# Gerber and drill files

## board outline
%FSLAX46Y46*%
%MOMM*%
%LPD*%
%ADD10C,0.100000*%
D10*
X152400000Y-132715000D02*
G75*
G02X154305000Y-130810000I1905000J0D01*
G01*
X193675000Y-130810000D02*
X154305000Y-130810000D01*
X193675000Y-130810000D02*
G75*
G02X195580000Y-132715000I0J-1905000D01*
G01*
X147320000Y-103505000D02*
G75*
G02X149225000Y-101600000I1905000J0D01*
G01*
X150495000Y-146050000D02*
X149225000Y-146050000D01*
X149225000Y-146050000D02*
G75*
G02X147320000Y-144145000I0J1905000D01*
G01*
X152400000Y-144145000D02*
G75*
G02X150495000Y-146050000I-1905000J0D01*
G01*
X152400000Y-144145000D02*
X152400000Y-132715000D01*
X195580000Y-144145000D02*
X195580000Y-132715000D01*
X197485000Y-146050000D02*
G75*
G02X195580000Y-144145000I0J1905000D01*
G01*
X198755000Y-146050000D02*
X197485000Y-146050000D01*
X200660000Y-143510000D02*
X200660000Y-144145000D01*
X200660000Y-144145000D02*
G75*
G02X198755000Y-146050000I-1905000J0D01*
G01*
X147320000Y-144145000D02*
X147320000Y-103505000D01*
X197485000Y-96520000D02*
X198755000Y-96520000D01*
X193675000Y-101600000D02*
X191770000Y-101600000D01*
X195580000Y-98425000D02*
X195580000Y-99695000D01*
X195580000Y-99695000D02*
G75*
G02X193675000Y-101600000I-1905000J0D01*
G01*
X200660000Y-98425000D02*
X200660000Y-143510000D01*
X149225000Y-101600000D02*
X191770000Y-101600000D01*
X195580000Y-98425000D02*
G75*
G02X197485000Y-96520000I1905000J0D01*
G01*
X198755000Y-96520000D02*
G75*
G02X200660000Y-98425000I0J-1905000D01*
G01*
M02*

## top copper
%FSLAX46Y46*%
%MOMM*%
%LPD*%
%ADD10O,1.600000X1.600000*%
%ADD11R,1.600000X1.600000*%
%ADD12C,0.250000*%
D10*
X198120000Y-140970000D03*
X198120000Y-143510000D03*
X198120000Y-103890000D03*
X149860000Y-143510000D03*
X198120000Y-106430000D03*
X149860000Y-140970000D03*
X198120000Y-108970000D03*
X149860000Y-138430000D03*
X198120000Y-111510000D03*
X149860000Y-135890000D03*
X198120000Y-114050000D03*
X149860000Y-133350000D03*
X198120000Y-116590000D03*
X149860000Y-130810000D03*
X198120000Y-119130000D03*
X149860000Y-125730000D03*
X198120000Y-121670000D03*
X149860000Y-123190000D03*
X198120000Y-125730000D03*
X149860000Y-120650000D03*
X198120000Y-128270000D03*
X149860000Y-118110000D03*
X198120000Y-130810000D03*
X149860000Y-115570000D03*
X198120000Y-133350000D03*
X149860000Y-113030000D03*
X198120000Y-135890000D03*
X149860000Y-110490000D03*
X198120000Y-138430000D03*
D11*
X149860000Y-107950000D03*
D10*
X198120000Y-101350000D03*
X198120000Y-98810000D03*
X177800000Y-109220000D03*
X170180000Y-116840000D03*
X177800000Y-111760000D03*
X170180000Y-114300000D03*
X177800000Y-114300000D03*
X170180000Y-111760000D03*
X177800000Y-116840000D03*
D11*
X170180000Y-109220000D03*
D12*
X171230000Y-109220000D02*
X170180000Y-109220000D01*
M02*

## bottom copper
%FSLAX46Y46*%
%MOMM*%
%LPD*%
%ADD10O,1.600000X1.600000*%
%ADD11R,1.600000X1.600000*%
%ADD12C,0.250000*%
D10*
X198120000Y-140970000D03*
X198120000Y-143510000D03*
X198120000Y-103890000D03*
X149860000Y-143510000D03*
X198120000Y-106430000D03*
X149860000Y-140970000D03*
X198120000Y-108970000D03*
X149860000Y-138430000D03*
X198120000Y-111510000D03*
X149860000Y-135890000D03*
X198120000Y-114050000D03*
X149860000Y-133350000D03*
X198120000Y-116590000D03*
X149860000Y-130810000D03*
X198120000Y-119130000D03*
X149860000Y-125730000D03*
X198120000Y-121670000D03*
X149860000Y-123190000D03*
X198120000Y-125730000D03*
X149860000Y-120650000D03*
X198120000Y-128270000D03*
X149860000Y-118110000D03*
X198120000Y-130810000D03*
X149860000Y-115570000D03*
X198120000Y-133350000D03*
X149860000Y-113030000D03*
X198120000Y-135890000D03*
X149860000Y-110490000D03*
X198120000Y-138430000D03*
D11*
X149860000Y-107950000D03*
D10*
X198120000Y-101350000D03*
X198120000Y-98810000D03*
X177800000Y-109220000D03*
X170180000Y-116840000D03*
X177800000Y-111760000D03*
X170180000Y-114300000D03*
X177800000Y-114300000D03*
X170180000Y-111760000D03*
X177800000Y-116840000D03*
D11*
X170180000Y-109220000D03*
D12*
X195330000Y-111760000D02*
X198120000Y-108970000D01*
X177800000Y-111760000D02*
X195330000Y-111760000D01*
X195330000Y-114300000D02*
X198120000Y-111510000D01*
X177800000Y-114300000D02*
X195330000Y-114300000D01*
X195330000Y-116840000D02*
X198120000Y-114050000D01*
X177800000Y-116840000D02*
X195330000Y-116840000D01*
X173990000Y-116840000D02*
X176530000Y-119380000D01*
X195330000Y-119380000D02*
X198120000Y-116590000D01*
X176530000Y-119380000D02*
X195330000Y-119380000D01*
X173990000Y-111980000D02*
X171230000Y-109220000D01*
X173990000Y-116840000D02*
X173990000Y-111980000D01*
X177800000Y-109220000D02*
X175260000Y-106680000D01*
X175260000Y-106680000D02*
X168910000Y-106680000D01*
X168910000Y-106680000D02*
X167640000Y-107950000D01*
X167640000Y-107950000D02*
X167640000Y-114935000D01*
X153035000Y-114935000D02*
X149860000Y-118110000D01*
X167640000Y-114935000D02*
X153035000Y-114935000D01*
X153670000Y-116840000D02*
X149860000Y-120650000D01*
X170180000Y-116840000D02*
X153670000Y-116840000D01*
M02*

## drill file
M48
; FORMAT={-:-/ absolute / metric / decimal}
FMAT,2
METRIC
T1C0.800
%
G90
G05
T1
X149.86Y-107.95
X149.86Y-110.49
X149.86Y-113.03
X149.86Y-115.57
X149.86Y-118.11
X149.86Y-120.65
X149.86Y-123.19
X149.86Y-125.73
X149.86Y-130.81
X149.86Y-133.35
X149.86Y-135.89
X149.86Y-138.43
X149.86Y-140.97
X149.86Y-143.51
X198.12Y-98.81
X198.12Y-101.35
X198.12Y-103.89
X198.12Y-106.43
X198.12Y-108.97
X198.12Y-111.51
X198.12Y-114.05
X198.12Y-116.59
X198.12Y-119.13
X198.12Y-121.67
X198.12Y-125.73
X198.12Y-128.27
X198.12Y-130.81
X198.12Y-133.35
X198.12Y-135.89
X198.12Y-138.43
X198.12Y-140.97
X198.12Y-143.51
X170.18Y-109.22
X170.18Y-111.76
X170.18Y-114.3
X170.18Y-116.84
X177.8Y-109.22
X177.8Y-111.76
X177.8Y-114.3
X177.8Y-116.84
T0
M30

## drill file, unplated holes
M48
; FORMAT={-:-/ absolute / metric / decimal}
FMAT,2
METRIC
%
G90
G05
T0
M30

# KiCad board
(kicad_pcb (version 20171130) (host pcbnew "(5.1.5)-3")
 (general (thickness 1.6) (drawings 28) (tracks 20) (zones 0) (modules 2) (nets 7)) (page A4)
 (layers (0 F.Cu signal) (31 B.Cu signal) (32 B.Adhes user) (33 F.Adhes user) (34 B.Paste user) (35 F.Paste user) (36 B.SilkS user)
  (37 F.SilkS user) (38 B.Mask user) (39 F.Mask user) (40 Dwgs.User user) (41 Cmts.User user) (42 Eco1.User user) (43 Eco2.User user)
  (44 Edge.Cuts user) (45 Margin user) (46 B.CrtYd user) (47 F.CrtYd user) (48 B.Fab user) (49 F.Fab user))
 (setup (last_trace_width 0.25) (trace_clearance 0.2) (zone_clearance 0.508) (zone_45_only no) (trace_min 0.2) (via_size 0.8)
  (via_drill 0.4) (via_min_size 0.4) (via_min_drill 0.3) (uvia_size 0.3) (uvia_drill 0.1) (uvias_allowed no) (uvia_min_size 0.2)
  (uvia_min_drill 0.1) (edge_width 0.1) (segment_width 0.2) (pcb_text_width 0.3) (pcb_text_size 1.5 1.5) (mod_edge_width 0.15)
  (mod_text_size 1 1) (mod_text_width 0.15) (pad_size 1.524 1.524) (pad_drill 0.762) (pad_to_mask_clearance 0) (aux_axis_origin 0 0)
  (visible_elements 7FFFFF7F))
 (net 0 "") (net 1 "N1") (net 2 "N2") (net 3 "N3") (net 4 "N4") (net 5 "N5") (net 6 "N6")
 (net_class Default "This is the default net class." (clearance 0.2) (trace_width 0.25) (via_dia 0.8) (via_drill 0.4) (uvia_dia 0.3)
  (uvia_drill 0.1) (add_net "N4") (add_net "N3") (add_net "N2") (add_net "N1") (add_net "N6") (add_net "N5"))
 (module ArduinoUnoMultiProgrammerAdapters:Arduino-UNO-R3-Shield (layer B.Cu) (at 149.86 107.95 270)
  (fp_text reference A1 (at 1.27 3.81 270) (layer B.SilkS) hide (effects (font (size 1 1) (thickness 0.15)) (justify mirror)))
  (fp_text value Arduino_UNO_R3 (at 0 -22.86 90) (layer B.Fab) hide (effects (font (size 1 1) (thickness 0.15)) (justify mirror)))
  (pad 16 thru_hole oval (at 33.02 -48.26 180) (size 1.6 1.6) (drill 0.8) (layers *.Cu *.Mask))
  (pad 15 thru_hole oval (at 35.56 -48.26 180) (size 1.6 1.6) (drill 0.8) (layers *.Cu *.Mask))
  (pad 30 thru_hole oval (at -4.06 -48.26 180) (size 1.6 1.6) (drill 0.8) (layers *.Cu *.Mask))
  (pad 14 thru_hole oval (at 35.56 0 180) (size 1.6 1.6) (drill 0.8) (layers *.Cu *.Mask))
  (pad 29 thru_hole oval (at -1.52 -48.26 180) (size 1.6 1.6) (drill 0.8) (layers *.Cu *.Mask))
  (pad 13 thru_hole oval (at 33.02 0 180) (size 1.6 1.6) (drill 0.8) (layers *.Cu *.Mask))
  (pad 28 thru_hole oval (at 1.02 -48.26 180) (size 1.6 1.6) (drill 0.8) (layers *.Cu *.Mask) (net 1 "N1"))
  (pad 12 thru_hole oval (at 30.48 0 180) (size 1.6 1.6) (drill 0.8) (layers *.Cu *.Mask))
  (pad 27 thru_hole oval (at 3.56 -48.26 180) (size 1.6 1.6) (drill 0.8) (layers *.Cu *.Mask) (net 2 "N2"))
  (pad 11 thru_hole oval (at 27.94 0 180) (size 1.6 1.6) (drill 0.8) (layers *.Cu *.Mask))
  (pad 26 thru_hole oval (at 6.1 -48.26 180) (size 1.6 1.6) (drill 0.8) (layers *.Cu *.Mask) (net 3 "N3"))
  (pad 10 thru_hole oval (at 25.4 0 180) (size 1.6 1.6) (drill 0.8) (layers *.Cu *.Mask))
  (pad 25 thru_hole oval (at 8.64 -48.26 180) (size 1.6 1.6) (drill 0.8) (layers *.Cu *.Mask) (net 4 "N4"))
  (pad 9 thru_hole oval (at 22.86 0 180) (size 1.6 1.6) (drill 0.8) (layers *.Cu *.Mask))
  (pad 24 thru_hole oval (at 11.18 -48.26 180) (size 1.6 1.6) (drill 0.8) (layers *.Cu *.Mask))
  (pad 8 thru_hole oval (at 17.78 0 180) (size 1.6 1.6) (drill 0.8) (layers *.Cu *.Mask))
  (pad 23 thru_hole oval (at 13.72 -48.26 180) (size 1.6 1.6) (drill 0.8) (layers *.Cu *.Mask))
  (pad 7 thru_hole oval (at 15.24 0 180) (size 1.6 1.6) (drill 0.8) (layers *.Cu *.Mask))
  (pad 22 thru_hole oval (at 17.78 -48.26 180) (size 1.6 1.6) (drill 0.8) (layers *.Cu *.Mask))
  (pad 6 thru_hole oval (at 12.7 0 180) (size 1.6 1.6) (drill 0.8) (layers *.Cu *.Mask) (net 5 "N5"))
  (pad 21 thru_hole oval (at 20.32 -48.26 180) (size 1.6 1.6) (drill 0.8) (layers *.Cu *.Mask))
  (pad 5 thru_hole oval (at 10.16 0 180) (size 1.6 1.6) (drill 0.8) (layers *.Cu *.Mask) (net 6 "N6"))
  (pad 20 thru_hole oval (at 22.86 -48.26 180) (size 1.6 1.6) (drill 0.8) (layers *.Cu *.Mask))
  (pad 4 thru_hole oval (at 7.62 0 180) (size 1.6 1.6) (drill 0.8) (layers *.Cu *.Mask))
  (pad 19 thru_hole oval (at 25.4 -48.26 180) (size 1.6 1.6) (drill 0.8) (layers *.Cu *.Mask))
  (pad 3 thru_hole oval (at 5.08 0 180) (size 1.6 1.6) (drill 0.8) (layers *.Cu *.Mask))
  (pad 18 thru_hole oval (at 27.94 -48.26 180) (size 1.6 1.6) (drill 0.8) (layers *.Cu *.Mask))
  (pad 2 thru_hole oval (at 2.54 0 180) (size 1.6 1.6) (drill 0.8) (layers *.Cu *.Mask))
  (pad 17 thru_hole oval (at 30.48 -48.26 180) (size 1.6 1.6) (drill 0.8) (layers *.Cu *.Mask))
  (pad 1 thru_hole rect (at 0 0 180) (size 1.6 1.6) (drill 0.8) (layers *.Cu *.Mask))
  (pad 31 thru_hole oval (at -6.6 -48.26 180) (size 1.6 1.6) (drill 0.8) (layers *.Cu *.Mask))
  (pad 32 thru_hole oval (at -9.14 -48.26 180) (size 1.6 1.6) (drill 0.8) (layers *.Cu *.Mask)))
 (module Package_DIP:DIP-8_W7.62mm (layer F.Cu) (at 170.18 109.22)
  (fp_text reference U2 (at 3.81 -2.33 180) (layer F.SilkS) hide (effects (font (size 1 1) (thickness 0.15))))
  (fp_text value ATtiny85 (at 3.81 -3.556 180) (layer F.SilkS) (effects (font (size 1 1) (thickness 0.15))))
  (pad 8 thru_hole oval (at 7.62 0) (size 1.6 1.6) (drill 0.8) (layers *.Cu *.Mask) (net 6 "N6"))
  (pad 4 thru_hole oval (at 0 7.62) (size 1.6 1.6) (drill 0.8) (layers *.Cu *.Mask) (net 5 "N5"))
  (pad 7 thru_hole oval (at 7.62 2.54) (size 1.6 1.6) (drill 0.8) (layers *.Cu *.Mask) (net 1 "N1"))
  (pad 3 thru_hole oval (at 0 5.08) (size 1.6 1.6) (drill 0.8) (layers *.Cu *.Mask))
  (pad 6 thru_hole oval (at 7.62 5.08) (size 1.6 1.6) (drill 0.8) (layers *.Cu *.Mask) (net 2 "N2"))
  (pad 2 thru_hole oval (at 0 2.54) (size 1.6 1.6) (drill 0.8) (layers *.Cu *.Mask))
  (pad 5 thru_hole oval (at 7.62 7.62) (size 1.6 1.6) (drill 0.8) (layers *.Cu *.Mask) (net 3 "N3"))
  (pad 1 thru_hole rect (at 0 0) (size 1.6 1.6) (drill 0.8) (layers *.Cu *.Mask) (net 4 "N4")))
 (gr_arc (start 154.305 132.715) (end 154.305 130.81) (angle -90) (layer Edge.Cuts) (width 0.1))
 (gr_line (start 193.675 130.81) (end 154.305 130.81) (layer Edge.Cuts) (width 0.1))
 (gr_arc (start 193.675 132.715) (end 195.58 132.715) (angle -90) (layer Edge.Cuts) (width 0.1))
 (gr_arc (start 149.225 103.505) (end 149.225 101.6) (angle -90) (layer Edge.Cuts) (width 0.1))
 (gr_line (start 150.495 146.05) (end 149.225 146.05) (layer Edge.Cuts) (width 0.1))
 (gr_arc (start 149.225 144.145) (end 147.32 144.145) (angle -90) (layer Edge.Cuts) (width 0.1))
 (gr_arc (start 150.495 144.145) (end 150.495 146.05) (angle -90) (layer Edge.Cuts) (width 0.1))
 (gr_line (start 152.4 144.145) (end 152.4 132.715) (layer Edge.Cuts) (width 0.1))
 (gr_line (start 195.58 144.145) (end 195.58 132.715) (layer Edge.Cuts) (width 0.1))
 (gr_arc (start 197.485 144.145) (end 195.58 144.145) (angle -90) (layer Edge.Cuts) (width 0.1))
 (gr_line (start 198.755 146.05) (end 197.485 146.05) (layer Edge.Cuts) (width 0.1))
 (gr_line (start 200.66 143.51) (end 200.66 144.145) (layer Edge.Cuts) (width 0.1))
 (gr_arc (start 198.755 144.145) (end 198.755 146.05) (angle -90) (layer Edge.Cuts) (width 0.1))
 (gr_line (start 147.32 144.145) (end 147.32 103.505) (layer Edge.Cuts) (width 0.1))
 (gr_line (start 197.485 96.52) (end 198.755 96.52) (layer Edge.Cuts) (width 0.1))
 (gr_line (start 193.675 101.6) (end 191.77 101.6) (layer Edge.Cuts) (width 0.1))
 (gr_line (start 195.58 98.425) (end 195.58 99.695) (layer Edge.Cuts) (width 0.1))
 (gr_arc (start 193.675 99.695) (end 193.675 101.6) (angle -90) (layer Edge.Cuts) (width 0.1))
 (gr_line (start 200.66 98.425) (end 200.66 143.51) (layer Edge.Cuts) (width 0.1))
 (gr_line (start 149.225 101.6) (end 191.77 101.6) (layer Edge.Cuts) (width 0.1))
 (gr_arc (start 197.485 98.425) (end 197.485 96.52) (angle -90) (layer Edge.Cuts) (width 0.1))
 (gr_arc (start 198.755 98.425) (end 200.66 98.425) (angle -90) (layer Edge.Cuts) (width 0.1))
 (segment (start 195.33 111.76) (end 198.12 108.97) (width 0.25) (layer B.Cu) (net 1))
 (segment (start 177.8 111.76) (end 195.33 111.76) (width 0.25) (layer B.Cu) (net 1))
 (segment (start 195.33 114.3) (end 198.12 111.51) (width 0.25) (layer B.Cu) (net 2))
 (segment (start 177.8 114.3) (end 195.33 114.3) (width 0.25) (layer B.Cu) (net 2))
 (segment (start 195.33 116.84) (end 198.12 114.05) (width 0.25) (layer B.Cu) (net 3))
 (segment (start 177.8 116.84) (end 195.33 116.84) (width 0.25) (layer B.Cu) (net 3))
 (segment (start 173.99 116.84) (end 176.53 119.38) (width 0.25) (layer B.Cu) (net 4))
 (segment (start 195.33 119.38) (end 198.12 116.59) (width 0.25) (layer B.Cu) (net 4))
 (segment (start 176.53 119.38) (end 195.33 119.38) (width 0.25) (layer B.Cu) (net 4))
 (segment (start 171.23 109.22) (end 170.18 109.22) (width 0.25) (layer F.Cu) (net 4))
 (segment (start 173.99 111.98) (end 171.23 109.22) (width 0.25) (layer B.Cu) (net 4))
 (segment (start 173.99 116.84) (end 173.99 111.98) (width 0.25) (layer B.Cu) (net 4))
 (segment (start 177.8 109.22) (end 175.26 106.68) (width 0.25) (layer B.Cu) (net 6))
 (segment (start 175.26 106.68) (end 168.91 106.68) (width 0.25) (layer B.Cu) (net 6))
 (segment (start 168.91 106.68) (end 167.64 107.95) (width 0.25) (layer B.Cu) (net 6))
 (segment (start 167.64 107.95) (end 167.64 114.935) (width 0.25) (layer B.Cu) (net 6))
 (segment (start 153.035 114.935) (end 149.86 118.11) (width 0.25) (layer B.Cu) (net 6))
 (segment (start 167.64 114.935) (end 153.035 114.935) (width 0.25) (layer B.Cu) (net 6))
 (segment (start 153.67 116.84) (end 149.86 120.65) (width 0.25) (layer B.Cu) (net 5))
 (segment (start 170.18 116.84) (end 153.67 116.84) (width 0.25) (layer B.Cu) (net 5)))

